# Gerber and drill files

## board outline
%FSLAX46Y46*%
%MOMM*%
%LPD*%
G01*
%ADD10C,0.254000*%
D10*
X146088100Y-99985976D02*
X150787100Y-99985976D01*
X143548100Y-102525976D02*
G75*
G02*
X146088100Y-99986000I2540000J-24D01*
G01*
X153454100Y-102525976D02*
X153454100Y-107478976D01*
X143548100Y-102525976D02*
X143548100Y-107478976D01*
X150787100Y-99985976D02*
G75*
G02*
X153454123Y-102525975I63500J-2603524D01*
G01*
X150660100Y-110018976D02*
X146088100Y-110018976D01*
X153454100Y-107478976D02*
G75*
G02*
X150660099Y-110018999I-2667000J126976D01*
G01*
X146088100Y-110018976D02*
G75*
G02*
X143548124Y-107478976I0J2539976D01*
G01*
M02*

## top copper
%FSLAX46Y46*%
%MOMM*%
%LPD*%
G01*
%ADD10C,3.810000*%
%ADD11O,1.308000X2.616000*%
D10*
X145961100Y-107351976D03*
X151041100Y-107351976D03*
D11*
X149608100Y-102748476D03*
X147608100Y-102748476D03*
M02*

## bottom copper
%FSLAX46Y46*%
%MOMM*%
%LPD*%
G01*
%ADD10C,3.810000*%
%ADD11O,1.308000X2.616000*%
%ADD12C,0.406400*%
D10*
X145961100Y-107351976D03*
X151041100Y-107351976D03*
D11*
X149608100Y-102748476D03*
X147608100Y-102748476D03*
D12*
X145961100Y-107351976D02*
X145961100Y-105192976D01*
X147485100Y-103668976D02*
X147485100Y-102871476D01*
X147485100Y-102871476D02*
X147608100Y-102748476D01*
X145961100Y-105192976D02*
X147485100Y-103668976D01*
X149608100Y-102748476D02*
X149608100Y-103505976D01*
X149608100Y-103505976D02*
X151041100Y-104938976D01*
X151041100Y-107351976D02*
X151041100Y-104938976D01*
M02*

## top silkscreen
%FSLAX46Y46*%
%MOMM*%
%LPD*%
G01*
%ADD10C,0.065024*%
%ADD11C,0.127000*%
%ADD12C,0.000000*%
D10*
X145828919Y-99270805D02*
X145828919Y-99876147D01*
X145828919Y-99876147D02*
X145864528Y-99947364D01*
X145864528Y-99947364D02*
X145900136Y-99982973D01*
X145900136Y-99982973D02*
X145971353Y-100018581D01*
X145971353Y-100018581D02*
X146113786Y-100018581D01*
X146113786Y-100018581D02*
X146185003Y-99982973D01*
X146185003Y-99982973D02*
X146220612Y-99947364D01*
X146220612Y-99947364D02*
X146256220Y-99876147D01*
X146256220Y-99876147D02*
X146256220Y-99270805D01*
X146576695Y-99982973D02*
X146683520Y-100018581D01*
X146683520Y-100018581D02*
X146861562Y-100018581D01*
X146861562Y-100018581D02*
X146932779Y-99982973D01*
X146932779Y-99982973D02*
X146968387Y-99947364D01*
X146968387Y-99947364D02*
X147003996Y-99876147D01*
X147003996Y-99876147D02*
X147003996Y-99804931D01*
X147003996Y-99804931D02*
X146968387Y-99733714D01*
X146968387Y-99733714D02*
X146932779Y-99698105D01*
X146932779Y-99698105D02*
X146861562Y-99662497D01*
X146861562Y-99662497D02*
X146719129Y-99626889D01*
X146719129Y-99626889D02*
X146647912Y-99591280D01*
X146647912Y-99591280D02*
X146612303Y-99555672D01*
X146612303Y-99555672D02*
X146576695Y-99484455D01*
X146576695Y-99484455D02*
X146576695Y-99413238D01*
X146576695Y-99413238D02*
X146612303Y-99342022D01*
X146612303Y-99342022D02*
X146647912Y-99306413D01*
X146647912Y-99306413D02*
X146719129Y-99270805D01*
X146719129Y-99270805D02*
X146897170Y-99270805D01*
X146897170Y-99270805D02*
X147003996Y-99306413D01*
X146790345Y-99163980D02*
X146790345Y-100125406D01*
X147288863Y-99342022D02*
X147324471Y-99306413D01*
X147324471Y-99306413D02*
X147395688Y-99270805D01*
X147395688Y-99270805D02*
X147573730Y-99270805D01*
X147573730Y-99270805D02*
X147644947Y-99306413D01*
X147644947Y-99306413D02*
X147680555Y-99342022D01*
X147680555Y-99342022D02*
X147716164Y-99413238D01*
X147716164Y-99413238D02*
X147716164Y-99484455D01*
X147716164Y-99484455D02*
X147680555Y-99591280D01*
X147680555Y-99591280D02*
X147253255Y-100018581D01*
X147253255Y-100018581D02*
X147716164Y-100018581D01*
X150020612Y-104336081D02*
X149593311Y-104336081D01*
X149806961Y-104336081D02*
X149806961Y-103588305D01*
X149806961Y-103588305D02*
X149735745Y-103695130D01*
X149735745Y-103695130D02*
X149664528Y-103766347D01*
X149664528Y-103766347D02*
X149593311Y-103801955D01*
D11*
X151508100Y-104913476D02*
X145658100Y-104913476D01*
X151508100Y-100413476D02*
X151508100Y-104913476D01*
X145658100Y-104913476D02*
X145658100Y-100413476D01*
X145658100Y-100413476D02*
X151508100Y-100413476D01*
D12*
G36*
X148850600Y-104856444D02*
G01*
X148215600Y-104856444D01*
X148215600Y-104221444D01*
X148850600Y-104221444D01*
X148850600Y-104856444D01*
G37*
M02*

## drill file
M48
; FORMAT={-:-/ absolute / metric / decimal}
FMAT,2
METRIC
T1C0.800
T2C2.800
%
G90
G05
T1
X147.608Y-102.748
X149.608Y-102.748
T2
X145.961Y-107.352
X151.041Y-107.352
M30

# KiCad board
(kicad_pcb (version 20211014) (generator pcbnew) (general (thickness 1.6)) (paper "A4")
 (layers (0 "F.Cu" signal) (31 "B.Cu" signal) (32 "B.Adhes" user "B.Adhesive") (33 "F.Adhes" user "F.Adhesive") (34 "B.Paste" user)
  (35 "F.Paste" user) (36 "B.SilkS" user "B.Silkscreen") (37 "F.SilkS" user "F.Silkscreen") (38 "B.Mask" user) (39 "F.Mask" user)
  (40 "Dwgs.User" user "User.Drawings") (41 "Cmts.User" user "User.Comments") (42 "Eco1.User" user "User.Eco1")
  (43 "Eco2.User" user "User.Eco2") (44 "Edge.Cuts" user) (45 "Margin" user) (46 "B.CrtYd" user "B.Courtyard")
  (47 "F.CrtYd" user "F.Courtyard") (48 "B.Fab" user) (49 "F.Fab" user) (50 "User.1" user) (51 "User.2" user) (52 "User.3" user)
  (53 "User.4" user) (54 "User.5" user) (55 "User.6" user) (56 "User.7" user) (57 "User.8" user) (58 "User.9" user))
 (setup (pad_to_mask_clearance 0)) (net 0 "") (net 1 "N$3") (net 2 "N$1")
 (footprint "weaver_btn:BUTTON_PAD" (layer "F.Cu") (at 145.9611 107.351976)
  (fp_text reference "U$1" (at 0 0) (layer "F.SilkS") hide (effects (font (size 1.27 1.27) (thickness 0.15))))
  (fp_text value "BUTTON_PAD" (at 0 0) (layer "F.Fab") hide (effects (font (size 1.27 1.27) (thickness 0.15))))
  (pad "P$1" thru_hole circle (at 0 0) (size 3.81 3.81) (drill 2.8) (layers *.Cu *.Mask) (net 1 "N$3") (solder_mask_margin 0.1016)))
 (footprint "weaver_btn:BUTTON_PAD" (layer "F.Cu") (at 151.0411 107.351976)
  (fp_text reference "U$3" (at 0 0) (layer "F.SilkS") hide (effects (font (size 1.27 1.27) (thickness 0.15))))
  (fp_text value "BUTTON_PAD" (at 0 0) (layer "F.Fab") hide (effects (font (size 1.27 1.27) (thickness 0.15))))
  (pad "P$1" thru_hole circle (at 0 0) (size 3.81 3.81) (drill 2.8) (layers *.Cu *.Mask) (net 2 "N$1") (solder_mask_margin 0.1016)))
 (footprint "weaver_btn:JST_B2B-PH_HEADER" (layer "F.Cu") (at 148.5331 102.795976)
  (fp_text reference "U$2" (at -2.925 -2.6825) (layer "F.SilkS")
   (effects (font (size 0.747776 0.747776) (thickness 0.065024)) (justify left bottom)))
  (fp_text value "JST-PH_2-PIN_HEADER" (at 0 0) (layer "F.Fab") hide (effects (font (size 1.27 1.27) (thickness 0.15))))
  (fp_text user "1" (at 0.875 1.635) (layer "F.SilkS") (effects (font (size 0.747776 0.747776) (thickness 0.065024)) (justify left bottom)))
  (fp_line (start 2.975 2.1175) (end -2.875 2.1175) (layer "F.SilkS") (width 0.127))
  (fp_line (start 2.975 -2.3825) (end 2.975 2.1175) (layer "F.SilkS") (width 0.127))
  (fp_line (start -2.875 2.1175) (end -2.875 -2.3825) (layer "F.SilkS") (width 0.127))
  (fp_line (start -2.875 -2.3825) (end 2.975 -2.3825) (layer "F.SilkS") (width 0.127))
  (fp_poly
   (pts (xy -0.3175 2.060468) (xy 0.3175 2.060468) (xy 0.3175 1.425468) (xy -0.3175 1.425468)) (layer "F.SilkS") (width 0) (fill solid))
  (pad "P1" thru_hole oval (at 1.075 -0.0475 90) (size 2.616 1.308) (drill 0.8) (layers *.Cu *.Mask) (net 2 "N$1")
   (solder_mask_margin 0.1016))
  (pad "P2" thru_hole oval (at -0.925 -0.0475 90) (size 2.616 1.308) (drill 0.8) (layers *.Cu *.Mask) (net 1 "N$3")
   (solder_mask_margin 0.1016)))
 (gr_line (start 146.0881 99.985976) (end 150.7871 99.985976) (layer "Edge.Cuts") (width 0.254))
 (gr_arc (start 143.5481 102.525976) (mid 144.292049 100.729925) (end 146.0881 99.985976) (layer "Edge.Cuts") (width 0.254))
 (gr_line (start 153.4541 102.525976) (end 153.4541 107.478976) (layer "Edge.Cuts") (width 0.254))
 (gr_line (start 143.5481 102.525976) (end 143.5481 107.478976) (layer "Edge.Cuts") (width 0.254))
 (gr_arc (start 150.7871 99.985976) (mid 152.646651 100.703622) (end 153.4541 102.525976) (layer "Edge.Cuts") (width 0.254))
 (gr_line (start 150.6601 110.018976) (end 146.0881 110.018976) (layer "Edge.Cuts") (width 0.254))
 (gr_arc (start 153.4541 107.478976) (mid 152.583151 109.327632) (end 150.6601 110.018976) (layer "Edge.Cuts") (width 0.254))
 (gr_arc (start 146.0881 110.018976) (mid 144.292049 109.275027) (end 143.5481 107.478976) (layer "Edge.Cuts") (width 0.254))
 (segment (start 145.9611 107.351976) (end 145.9611 105.192976) (width 0.4064) (layer "B.Cu") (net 1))
 (segment (start 147.4851 103.668976) (end 147.4851 102.871476) (width 0.4064) (layer "B.Cu") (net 1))
 (segment (start 147.4851 102.871476) (end 147.6081 102.748476) (width 0.4064) (layer "B.Cu") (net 1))
 (segment (start 145.9611 105.192976) (end 147.4851 103.668976) (width 0.4064) (layer "B.Cu") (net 1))
 (segment (start 149.6081 102.748476) (end 149.6081 103.505976) (width 0.4064) (layer "B.Cu") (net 2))
 (segment (start 149.6081 103.505976) (end 151.0411 104.938976) (width 0.4064) (layer "B.Cu") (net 2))
 (segment (start 151.0411 107.351976) (end 151.0411 104.938976) (width 0.4064) (layer "B.Cu") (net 2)))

